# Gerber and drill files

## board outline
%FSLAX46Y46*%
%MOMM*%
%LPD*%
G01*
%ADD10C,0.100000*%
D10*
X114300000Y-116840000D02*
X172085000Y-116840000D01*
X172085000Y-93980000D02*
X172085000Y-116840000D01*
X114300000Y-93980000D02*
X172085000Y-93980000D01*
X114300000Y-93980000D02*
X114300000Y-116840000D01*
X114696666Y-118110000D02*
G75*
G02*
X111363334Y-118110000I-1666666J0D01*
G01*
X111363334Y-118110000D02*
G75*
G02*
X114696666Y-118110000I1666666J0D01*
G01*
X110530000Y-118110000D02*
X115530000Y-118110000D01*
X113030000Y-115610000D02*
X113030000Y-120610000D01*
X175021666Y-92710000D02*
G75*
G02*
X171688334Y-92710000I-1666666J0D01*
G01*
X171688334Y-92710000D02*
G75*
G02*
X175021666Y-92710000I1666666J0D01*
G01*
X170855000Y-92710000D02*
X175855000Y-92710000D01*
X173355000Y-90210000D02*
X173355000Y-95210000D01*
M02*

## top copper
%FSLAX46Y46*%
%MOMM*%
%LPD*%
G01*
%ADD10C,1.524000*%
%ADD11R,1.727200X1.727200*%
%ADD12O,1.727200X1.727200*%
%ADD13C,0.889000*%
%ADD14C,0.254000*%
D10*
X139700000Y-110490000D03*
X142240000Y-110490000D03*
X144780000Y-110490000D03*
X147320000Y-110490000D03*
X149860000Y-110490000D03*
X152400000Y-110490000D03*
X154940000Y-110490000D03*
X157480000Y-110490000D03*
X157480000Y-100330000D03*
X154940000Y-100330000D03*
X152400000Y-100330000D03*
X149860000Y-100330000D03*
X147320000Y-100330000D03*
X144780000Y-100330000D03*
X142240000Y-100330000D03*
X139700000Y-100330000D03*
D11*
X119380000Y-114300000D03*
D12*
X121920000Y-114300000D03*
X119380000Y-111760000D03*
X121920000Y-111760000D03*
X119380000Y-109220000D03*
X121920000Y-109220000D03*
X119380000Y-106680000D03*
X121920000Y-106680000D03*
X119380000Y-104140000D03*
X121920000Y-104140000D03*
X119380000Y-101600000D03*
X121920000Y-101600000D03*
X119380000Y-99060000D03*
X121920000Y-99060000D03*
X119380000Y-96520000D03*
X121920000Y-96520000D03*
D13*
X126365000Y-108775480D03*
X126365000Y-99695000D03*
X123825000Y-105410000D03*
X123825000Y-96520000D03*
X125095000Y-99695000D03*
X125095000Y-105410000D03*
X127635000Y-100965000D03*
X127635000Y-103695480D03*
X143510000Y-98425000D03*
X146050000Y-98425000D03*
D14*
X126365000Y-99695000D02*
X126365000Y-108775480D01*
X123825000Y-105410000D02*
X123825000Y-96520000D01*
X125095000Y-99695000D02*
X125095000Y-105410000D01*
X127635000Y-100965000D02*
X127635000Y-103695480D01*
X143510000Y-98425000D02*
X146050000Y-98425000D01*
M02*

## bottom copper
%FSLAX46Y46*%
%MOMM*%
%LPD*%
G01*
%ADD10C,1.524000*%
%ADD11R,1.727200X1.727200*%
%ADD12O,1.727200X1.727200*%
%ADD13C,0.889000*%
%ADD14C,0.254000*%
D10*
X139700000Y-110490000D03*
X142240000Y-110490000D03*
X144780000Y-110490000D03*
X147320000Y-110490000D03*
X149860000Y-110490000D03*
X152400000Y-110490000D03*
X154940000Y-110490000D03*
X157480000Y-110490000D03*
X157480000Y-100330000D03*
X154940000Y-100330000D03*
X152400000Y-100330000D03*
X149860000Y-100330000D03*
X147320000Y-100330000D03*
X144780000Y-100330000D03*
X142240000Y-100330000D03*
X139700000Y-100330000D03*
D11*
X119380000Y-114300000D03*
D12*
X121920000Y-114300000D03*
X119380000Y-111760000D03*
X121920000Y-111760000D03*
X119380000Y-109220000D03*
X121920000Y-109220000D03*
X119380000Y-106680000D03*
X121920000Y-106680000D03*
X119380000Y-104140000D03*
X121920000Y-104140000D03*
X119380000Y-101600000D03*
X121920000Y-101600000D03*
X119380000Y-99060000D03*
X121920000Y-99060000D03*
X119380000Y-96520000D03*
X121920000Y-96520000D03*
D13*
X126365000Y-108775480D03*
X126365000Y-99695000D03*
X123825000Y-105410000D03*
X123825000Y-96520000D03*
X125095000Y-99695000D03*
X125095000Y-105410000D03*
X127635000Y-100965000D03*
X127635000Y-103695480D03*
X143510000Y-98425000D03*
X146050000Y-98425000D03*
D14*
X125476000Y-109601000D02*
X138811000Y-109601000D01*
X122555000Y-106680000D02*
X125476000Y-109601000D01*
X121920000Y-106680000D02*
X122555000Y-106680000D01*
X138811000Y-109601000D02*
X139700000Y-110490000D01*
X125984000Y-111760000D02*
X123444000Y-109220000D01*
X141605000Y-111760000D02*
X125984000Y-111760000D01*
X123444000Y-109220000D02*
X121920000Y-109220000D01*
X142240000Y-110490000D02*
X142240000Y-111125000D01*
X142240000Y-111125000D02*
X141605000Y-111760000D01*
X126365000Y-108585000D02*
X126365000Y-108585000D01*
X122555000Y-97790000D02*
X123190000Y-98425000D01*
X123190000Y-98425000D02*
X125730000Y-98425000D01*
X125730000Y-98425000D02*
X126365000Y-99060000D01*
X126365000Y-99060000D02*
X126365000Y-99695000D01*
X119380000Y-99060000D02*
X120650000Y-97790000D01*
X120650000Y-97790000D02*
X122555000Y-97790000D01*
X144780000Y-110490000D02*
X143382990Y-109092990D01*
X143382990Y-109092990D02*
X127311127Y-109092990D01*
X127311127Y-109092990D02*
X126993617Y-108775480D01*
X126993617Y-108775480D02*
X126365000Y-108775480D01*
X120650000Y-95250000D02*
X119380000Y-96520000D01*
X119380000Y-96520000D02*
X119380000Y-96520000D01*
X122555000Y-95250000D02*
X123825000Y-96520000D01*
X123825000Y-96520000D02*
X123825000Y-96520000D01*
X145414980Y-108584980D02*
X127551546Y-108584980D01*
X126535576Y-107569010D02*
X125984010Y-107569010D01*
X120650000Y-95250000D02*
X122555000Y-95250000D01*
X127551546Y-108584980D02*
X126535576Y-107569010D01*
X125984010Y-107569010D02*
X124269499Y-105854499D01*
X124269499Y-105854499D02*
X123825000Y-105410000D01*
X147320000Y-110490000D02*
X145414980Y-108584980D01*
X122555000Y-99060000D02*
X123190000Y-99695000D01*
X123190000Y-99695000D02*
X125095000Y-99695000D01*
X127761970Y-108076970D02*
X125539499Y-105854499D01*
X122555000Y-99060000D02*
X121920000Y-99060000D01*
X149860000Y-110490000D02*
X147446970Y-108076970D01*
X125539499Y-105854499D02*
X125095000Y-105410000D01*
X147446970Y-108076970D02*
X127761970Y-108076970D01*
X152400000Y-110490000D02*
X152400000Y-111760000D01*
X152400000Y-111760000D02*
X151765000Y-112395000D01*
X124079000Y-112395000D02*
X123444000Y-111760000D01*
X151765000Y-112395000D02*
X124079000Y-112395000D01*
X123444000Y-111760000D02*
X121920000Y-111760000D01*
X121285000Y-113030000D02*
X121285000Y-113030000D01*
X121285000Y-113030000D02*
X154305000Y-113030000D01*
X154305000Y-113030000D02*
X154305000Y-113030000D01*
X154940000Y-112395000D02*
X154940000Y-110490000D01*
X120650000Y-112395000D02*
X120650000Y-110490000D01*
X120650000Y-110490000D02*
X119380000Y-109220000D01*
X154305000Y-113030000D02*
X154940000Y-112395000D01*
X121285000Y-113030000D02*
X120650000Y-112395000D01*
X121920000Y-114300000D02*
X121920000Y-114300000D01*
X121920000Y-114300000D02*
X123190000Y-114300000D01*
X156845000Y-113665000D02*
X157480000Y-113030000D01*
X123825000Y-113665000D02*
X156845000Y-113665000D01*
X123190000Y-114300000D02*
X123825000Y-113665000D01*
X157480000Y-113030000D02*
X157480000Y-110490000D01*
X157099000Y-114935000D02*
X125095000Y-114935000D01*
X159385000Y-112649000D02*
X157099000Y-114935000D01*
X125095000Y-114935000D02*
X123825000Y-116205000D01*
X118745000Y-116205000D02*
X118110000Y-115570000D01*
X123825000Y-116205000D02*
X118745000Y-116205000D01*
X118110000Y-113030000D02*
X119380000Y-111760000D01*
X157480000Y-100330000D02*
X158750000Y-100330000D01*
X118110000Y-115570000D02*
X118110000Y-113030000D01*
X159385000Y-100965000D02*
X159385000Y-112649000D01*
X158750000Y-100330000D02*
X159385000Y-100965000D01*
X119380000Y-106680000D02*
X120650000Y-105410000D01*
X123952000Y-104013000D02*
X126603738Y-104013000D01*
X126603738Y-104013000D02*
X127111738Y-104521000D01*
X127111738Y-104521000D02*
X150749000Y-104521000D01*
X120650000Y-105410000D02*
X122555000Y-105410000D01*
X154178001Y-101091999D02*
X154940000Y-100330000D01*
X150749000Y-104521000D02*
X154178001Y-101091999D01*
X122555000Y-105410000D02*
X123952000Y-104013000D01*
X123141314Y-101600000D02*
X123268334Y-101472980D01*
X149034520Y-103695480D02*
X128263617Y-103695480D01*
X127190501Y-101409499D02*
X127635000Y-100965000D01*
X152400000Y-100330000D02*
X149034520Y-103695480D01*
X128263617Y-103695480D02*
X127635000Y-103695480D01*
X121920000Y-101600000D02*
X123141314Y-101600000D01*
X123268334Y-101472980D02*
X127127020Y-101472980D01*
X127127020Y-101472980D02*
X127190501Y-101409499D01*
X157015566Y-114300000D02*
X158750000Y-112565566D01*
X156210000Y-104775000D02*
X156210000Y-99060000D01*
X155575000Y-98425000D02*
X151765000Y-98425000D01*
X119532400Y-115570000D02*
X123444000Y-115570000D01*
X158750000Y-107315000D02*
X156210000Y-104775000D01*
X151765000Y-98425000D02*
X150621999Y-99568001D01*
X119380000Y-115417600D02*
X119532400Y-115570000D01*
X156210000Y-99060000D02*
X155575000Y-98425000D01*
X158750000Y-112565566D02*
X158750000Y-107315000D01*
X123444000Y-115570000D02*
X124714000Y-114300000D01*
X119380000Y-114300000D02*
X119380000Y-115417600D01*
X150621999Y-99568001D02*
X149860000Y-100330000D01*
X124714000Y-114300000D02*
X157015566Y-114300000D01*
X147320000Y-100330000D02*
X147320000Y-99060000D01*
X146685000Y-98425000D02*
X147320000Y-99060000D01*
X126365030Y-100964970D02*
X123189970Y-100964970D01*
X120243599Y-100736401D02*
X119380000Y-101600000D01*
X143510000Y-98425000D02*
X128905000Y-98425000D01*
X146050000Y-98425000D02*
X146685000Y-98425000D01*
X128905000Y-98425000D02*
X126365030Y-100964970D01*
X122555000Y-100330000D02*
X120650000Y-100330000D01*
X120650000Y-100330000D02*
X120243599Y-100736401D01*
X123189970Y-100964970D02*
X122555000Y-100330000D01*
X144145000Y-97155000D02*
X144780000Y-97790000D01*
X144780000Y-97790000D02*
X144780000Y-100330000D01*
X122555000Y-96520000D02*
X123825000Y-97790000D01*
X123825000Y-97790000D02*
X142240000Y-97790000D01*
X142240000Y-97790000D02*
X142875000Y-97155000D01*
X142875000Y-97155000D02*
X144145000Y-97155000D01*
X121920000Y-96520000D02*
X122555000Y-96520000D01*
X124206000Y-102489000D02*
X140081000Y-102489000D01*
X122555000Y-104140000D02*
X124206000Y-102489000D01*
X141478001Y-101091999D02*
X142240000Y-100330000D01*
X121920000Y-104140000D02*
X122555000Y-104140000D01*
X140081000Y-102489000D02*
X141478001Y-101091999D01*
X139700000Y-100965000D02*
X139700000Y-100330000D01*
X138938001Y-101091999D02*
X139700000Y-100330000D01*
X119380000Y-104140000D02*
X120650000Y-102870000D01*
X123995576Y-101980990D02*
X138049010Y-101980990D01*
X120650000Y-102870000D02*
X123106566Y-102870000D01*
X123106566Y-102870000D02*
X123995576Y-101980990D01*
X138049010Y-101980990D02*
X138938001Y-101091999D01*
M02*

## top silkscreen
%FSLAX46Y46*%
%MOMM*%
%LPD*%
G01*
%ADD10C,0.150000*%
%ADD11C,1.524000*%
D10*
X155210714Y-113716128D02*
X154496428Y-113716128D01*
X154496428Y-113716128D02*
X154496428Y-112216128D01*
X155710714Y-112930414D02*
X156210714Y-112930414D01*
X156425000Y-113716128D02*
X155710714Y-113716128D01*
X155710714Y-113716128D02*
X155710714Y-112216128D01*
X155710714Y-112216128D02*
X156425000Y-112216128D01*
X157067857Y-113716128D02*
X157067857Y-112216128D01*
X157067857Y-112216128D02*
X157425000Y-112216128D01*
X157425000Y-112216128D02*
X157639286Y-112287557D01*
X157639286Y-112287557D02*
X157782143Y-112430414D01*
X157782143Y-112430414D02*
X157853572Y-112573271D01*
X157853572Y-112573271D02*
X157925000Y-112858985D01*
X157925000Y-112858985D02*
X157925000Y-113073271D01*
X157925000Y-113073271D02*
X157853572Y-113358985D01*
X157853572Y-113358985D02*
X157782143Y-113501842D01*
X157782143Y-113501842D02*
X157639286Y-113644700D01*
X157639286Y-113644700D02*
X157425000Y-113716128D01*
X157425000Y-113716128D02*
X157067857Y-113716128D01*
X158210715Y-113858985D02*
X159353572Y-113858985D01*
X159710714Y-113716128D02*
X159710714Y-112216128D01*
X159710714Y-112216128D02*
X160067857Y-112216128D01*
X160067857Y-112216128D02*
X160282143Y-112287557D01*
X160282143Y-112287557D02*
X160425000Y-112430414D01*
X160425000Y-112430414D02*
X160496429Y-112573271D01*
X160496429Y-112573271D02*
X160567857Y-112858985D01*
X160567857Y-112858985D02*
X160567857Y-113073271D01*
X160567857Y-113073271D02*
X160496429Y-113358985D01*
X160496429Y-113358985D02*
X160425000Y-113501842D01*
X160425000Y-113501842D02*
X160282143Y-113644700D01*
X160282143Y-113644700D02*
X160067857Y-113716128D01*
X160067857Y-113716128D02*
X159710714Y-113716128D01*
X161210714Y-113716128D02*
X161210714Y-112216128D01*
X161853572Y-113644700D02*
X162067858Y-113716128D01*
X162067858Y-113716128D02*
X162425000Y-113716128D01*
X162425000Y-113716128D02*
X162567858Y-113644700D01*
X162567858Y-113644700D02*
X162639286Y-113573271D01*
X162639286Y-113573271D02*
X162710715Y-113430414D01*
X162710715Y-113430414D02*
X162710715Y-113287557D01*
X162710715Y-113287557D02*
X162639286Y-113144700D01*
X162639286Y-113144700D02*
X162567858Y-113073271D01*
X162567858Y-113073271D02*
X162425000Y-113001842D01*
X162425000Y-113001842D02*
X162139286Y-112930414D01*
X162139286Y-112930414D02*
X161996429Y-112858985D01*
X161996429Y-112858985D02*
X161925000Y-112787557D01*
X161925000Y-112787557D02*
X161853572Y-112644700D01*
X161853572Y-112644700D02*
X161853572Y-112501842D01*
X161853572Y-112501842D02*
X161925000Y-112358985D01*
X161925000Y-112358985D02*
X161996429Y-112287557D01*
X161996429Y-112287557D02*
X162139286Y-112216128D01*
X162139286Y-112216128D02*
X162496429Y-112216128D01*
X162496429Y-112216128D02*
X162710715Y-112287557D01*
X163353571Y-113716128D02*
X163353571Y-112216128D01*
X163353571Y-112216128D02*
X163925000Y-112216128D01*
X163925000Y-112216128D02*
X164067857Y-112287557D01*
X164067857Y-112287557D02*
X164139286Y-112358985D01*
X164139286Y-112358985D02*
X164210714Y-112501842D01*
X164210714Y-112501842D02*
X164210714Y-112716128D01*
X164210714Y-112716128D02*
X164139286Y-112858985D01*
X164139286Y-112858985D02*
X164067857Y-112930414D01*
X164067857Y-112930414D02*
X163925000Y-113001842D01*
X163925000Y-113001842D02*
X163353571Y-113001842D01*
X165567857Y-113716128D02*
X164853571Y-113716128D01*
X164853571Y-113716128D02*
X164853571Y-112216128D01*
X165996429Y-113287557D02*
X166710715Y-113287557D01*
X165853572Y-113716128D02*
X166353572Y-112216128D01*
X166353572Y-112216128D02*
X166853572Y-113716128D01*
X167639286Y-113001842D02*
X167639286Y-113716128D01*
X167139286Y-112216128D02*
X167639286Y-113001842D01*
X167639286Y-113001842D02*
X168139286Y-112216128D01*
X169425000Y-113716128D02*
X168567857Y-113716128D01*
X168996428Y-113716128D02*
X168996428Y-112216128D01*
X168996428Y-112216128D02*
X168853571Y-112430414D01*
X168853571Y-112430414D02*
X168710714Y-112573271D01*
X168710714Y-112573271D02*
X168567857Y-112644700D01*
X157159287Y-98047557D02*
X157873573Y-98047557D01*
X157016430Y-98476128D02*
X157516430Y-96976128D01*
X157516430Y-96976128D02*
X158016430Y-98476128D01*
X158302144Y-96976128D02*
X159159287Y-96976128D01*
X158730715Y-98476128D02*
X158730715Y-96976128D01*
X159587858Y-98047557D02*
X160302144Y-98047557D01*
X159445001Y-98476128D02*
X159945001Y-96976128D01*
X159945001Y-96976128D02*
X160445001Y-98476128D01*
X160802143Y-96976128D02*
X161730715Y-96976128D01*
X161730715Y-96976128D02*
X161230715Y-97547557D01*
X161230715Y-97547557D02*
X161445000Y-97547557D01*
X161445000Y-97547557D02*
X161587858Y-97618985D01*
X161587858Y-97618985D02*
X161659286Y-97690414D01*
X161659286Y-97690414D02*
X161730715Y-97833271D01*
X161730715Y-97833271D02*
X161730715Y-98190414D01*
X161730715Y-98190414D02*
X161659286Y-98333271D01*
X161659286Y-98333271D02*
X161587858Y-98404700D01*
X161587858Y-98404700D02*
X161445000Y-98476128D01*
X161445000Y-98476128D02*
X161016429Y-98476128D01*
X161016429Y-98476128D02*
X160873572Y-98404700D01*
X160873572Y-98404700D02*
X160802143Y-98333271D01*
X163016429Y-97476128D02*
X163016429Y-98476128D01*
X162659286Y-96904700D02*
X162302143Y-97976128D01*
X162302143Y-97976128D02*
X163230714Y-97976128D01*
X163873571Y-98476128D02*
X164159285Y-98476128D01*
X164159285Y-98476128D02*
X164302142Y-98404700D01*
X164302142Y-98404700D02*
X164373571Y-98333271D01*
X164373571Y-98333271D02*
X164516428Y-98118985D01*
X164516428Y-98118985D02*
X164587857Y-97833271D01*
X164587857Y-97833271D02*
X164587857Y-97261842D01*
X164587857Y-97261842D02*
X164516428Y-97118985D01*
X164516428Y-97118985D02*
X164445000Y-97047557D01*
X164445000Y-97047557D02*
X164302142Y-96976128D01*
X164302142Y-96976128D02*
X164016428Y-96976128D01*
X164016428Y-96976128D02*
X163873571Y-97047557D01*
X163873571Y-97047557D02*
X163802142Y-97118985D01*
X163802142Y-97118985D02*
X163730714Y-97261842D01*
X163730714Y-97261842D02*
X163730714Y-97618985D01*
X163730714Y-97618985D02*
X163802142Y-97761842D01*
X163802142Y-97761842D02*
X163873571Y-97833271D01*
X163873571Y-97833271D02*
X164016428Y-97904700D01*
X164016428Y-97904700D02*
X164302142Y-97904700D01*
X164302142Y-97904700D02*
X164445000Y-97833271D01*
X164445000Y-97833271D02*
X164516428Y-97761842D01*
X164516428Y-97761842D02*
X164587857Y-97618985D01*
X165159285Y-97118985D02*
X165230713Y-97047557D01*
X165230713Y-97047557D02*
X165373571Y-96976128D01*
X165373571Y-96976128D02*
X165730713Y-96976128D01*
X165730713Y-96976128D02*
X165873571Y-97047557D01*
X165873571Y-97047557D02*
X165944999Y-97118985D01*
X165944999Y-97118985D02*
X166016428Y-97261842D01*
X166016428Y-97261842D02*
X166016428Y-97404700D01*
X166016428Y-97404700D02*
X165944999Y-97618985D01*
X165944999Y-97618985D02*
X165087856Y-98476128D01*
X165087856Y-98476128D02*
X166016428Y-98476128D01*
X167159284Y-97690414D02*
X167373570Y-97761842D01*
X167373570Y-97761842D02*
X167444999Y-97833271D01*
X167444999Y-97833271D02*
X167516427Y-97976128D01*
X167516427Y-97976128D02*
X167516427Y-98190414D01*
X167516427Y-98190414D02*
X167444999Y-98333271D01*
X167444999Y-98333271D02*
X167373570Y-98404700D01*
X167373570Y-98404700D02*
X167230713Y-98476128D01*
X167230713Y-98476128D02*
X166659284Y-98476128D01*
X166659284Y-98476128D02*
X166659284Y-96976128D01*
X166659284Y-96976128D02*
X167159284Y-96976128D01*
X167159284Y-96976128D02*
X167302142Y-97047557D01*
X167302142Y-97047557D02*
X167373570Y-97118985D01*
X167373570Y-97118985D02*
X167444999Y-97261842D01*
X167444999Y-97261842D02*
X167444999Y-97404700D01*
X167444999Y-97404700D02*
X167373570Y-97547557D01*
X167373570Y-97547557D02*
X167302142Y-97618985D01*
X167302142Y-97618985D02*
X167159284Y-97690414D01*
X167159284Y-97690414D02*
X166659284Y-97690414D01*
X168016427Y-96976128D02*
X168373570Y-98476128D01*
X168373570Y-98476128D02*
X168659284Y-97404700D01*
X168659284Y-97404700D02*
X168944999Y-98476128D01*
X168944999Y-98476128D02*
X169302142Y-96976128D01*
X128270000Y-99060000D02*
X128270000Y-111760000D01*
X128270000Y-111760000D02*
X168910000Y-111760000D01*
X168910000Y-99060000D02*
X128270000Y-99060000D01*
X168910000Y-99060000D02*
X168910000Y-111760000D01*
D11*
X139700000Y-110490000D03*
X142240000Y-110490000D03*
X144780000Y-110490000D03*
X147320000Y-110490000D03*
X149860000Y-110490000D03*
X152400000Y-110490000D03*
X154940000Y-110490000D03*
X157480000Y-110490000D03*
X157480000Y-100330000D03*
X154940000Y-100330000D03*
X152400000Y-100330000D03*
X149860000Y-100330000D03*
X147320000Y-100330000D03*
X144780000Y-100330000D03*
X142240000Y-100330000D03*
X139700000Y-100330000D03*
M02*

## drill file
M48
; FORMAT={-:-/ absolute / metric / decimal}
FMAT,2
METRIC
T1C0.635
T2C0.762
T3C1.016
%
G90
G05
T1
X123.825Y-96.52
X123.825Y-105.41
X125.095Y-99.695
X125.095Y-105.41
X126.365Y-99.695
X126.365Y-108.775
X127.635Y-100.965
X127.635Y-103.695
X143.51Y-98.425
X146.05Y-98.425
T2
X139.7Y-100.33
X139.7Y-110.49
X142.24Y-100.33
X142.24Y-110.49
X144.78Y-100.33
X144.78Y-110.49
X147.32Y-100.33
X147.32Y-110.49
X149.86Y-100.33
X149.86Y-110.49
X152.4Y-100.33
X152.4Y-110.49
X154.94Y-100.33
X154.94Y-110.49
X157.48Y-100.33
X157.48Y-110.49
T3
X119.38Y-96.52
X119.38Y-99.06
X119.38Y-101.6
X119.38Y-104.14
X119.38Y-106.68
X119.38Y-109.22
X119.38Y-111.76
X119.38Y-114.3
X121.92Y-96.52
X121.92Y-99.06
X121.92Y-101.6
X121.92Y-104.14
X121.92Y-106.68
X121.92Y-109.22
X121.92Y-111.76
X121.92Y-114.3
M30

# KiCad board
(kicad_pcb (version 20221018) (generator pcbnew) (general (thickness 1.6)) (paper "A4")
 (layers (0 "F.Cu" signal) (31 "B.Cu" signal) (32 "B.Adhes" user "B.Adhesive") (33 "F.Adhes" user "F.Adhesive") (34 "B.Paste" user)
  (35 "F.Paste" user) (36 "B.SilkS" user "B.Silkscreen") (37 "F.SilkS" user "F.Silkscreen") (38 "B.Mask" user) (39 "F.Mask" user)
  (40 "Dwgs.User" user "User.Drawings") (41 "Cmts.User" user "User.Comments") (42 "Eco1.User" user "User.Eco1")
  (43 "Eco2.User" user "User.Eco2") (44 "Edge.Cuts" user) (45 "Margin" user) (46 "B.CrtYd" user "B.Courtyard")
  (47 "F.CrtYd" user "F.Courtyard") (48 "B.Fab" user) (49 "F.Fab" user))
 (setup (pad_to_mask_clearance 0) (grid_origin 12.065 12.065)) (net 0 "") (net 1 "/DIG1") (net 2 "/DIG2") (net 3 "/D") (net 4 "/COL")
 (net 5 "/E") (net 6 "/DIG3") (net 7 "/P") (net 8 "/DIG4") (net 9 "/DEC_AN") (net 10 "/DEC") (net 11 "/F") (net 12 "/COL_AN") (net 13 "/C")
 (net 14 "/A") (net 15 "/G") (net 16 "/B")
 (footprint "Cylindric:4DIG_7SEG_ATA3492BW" (layer "F.Cu") (at 148.59 105.41)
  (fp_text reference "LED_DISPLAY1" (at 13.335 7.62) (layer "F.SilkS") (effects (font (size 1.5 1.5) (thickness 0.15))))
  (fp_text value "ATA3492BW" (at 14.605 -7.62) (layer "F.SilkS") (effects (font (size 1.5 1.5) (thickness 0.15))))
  (fp_line (start -20.32 -6.35) (end -20.32 6.35) (stroke (width 0.15) (type solid)) (layer "F.SilkS"))
  (fp_line (start -20.32 6.35) (end 20.32 6.35) (stroke (width 0.15) (type solid)) (layer "F.SilkS"))
  (fp_line (start 20.32 -6.35) (end -20.32 -6.35) (stroke (width 0.15) (type solid)) (layer "F.SilkS"))
  (fp_line (start 20.32 -6.35) (end 20.32 6.35) (stroke (width 0.15) (type solid)) (layer "F.SilkS"))
  (pad "1" thru_hole circle (at -8.89 5.08) (size 1.524 1.524) (drill 0.762) (layers "*.Cu" "*.Mask" "F.SilkS") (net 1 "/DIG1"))
  (pad "2" thru_hole circle (at -6.35 5.08) (size 1.524 1.524) (drill 0.762) (layers "*.Cu" "*.Mask" "F.SilkS") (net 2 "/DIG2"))
  (pad "3" thru_hole circle (at -3.81 5.08) (size 1.524 1.524) (drill 0.762) (layers "*.Cu" "*.Mask" "F.SilkS") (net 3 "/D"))
  (pad "4" thru_hole circle (at -1.27 5.08) (size 1.524 1.524) (drill 0.762) (layers "*.Cu" "*.Mask" "F.SilkS") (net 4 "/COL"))
  (pad "5" thru_hole circle (at 1.27 5.08) (size 1.524 1.524) (drill 0.762) (layers "*.Cu" "*.Mask" "F.SilkS") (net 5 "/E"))
  (pad "6" thru_hole circle (at 3.81 5.08) (size 1.524 1.524) (drill 0.762) (layers "*.Cu" "*.Mask" "F.SilkS") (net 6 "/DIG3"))
  (pad "7" thru_hole circle (at 6.35 5.08) (size 1.524 1.524) (drill 0.762) (layers "*.Cu" "*.Mask" "F.SilkS") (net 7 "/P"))
  (pad "8" thru_hole circle (at 8.89 5.08) (size 1.524 1.524) (drill 0.762) (layers "*.Cu" "*.Mask" "F.SilkS") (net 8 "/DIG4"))
  (pad "9" thru_hole circle (at 8.89 -5.08) (size 1.524 1.524) (drill 0.762) (layers "*.Cu" "*.Mask" "F.SilkS") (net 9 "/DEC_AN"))
  (pad "10" thru_hole circle (at 6.35 -5.08) (size 1.524 1.524) (drill 0.762) (layers "*.Cu" "*.Mask" "F.SilkS") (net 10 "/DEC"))
  (pad "11" thru_hole circle (at 3.81 -5.08) (size 1.524 1.524) (drill 0.762) (layers "*.Cu" "*.Mask" "F.SilkS") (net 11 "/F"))
  (pad "12" thru_hole circle (at 1.27 -5.08) (size 1.524 1.524) (drill 0.762) (layers "*.Cu" "*.Mask" "F.SilkS") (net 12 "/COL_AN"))
  (pad "13" thru_hole circle (at -1.27 -5.08) (size 1.524 1.524) (drill 0.762) (layers "*.Cu" "*.Mask" "F.SilkS") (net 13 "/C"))
  (pad "14" thru_hole circle (at -3.81 -5.08) (size 1.524 1.524) (drill 0.762) (layers "*.Cu" "*.Mask" "F.SilkS") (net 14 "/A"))
  (pad "15" thru_hole circle (at -6.35 -5.08) (size 1.524 1.524) (drill 0.762) (layers "*.Cu" "*.Mask" "F.SilkS") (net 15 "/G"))
  (pad "16" thru_hole circle (at -8.89 -5.08) (size 1.524 1.524) (drill 0.762) (layers "*.Cu" "*.Mask" "F.SilkS") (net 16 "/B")))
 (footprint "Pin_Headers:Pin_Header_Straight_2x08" (layer "B.Cu") (at 120.65 105.41 90)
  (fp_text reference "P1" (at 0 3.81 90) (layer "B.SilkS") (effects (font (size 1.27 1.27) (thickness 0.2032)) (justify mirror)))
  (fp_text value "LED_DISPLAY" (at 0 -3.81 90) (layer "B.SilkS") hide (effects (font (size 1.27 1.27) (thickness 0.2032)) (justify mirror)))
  (pad "1" thru_hole rect (at -8.89 -1.27 90) (size 1.7272 1.7272) (drill 1.016) (layers "*.Cu" "*.Mask" "B.SilkS") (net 12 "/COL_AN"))
  (pad "2" thru_hole oval (at -8.89 1.27 90) (size 1.7272 1.7272) (drill 1.016) (layers "*.Cu" "*.Mask" "B.SilkS") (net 8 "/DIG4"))
  (pad "3" thru_hole oval (at -6.35 -1.27 90) (size 1.7272 1.7272) (drill 1.016) (layers "*.Cu" "*.Mask" "B.SilkS") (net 9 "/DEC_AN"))
  (pad "4" thru_hole oval (at -6.35 1.27 90) (size 1.7272 1.7272) (drill 1.016) (layers "*.Cu" "*.Mask" "B.SilkS") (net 6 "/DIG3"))
  (pad "5" thru_hole oval (at -3.81 -1.27 90) (size 1.7272 1.7272) (drill 1.016) (layers "*.Cu" "*.Mask" "B.SilkS") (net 7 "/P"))
  (pad "6" thru_hole oval (at -3.81 1.27 90) (size 1.7272 1.7272) (drill 1.016) (layers "*.Cu" "*.Mask" "B.SilkS") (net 2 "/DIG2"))
  (pad "7" thru_hole oval (at -1.27 -1.27 90) (size 1.7272 1.7272) (drill 1.016) (layers "*.Cu" "*.Mask" "B.SilkS") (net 10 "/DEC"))
  (pad "8" thru_hole oval (at -1.27 1.27 90) (size 1.7272 1.7272) (drill 1.016) (layers "*.Cu" "*.Mask" "B.SilkS") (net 1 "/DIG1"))
  (pad "9" thru_hole oval (at 1.27 -1.27 90) (size 1.7272 1.7272) (drill 1.016) (layers "*.Cu" "*.Mask" "B.SilkS") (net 16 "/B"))
  (pad "10" thru_hole oval (at 1.27 1.27 90) (size 1.7272 1.7272) (drill 1.016) (layers "*.Cu" "*.Mask" "B.SilkS") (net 15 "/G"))
  (pad "11" thru_hole oval (at 3.81 -1.27 90) (size 1.7272 1.7272) (drill 1.016) (layers "*.Cu" "*.Mask" "B.SilkS") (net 13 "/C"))
  (pad "12" thru_hole oval (at 3.81 1.27 90) (size 1.7272 1.7272) (drill 1.016) (layers "*.Cu" "*.Mask" "B.SilkS") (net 11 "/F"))
  (pad "13" thru_hole oval (at 6.35 -1.27 90) (size 1.7272 1.7272) (drill 1.016) (layers "*.Cu" "*.Mask" "B.SilkS") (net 3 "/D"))
  (pad "14" thru_hole oval (at 6.35 1.27 90) (size 1.7272 1.7272) (drill 1.016) (layers "*.Cu" "*.Mask" "B.SilkS") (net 5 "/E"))
  (pad "15" thru_hole oval (at 8.89 -1.27 90) (size 1.7272 1.7272) (drill 1.016) (layers "*.Cu" "*.Mask" "B.SilkS") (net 4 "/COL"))
  (pad "16" thru_hole oval (at 8.89 1.27 90) (size 1.7272 1.7272) (drill 1.016) (layers "*.Cu" "*.Mask" "B.SilkS") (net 14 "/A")))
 (gr_line (start 114.3 116.84) (end 172.085 116.84) (stroke (width 0.1) (type solid)) (layer "Edge.Cuts"))
 (gr_line (start 172.085 93.98) (end 172.085 116.84) (stroke (width 0.1) (type solid)) (layer "Edge.Cuts"))
 (gr_line (start 114.3 93.98) (end 172.085 93.98) (stroke (width 0.1) (type solid)) (layer "Edge.Cuts"))
 (gr_line (start 114.3 93.98) (end 114.3 116.84) (stroke (width 0.1) (type solid)) (layer "Edge.Cuts"))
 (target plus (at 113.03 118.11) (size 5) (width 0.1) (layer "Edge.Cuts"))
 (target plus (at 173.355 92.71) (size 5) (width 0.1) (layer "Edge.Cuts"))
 (segment (start 125.476 109.601) (end 138.811 109.601) (width 0.254) (layer "B.Cu") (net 1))
 (segment (start 122.555 106.68) (end 125.476 109.601) (width 0.254) (layer "B.Cu") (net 1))
 (segment (start 121.92 106.68) (end 122.555 106.68) (width 0.254) (layer "B.Cu") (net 1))
 (segment (start 138.811 109.601) (end 139.7 110.49) (width 0.254) (layer "B.Cu") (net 1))
 (segment (start 125.984 111.76) (end 123.444 109.22) (width 0.254) (layer "B.Cu") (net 2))
 (segment (start 141.605 111.76) (end 125.984 111.76) (width 0.254) (layer "B.Cu") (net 2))
 (segment (start 123.444 109.22) (end 121.92 109.22) (width 0.254) (layer "B.Cu") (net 2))
 (segment (start 142.24 110.49) (end 142.24 111.125) (width 0.254) (layer "B.Cu") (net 2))
 (segment (start 142.24 111.125) (end 141.605 111.76) (width 0.254) (layer "B.Cu") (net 2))
 (segment (start 126.365 99.695) (end 126.365 108.77548) (width 0.254) (layer "F.Cu") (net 3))
 (via (at 126.365 108.77548) (size 0.889) (drill 0.635) (layers "F.Cu" "B.Cu") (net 3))
 (via (at 126.365 99.695) (size 0.889) (drill 0.635) (layers "F.Cu" "B.Cu") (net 3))
 (segment (start 126.365 108.585) (end 126.365 108.585) (width 0.254) (layer "B.Cu") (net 3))
 (segment (start 122.555 97.79) (end 123.19 98.425) (width 0.254) (layer "B.Cu") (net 3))
 (segment (start 123.19 98.425) (end 125.73 98.425) (width 0.254) (layer "B.Cu") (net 3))
 (segment (start 125.73 98.425) (end 126.365 99.06) (width 0.254) (layer "B.Cu") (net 3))
 (segment (start 126.365 99.06) (end 126.365 99.695) (width 0.254) (layer "B.Cu") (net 3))
 (segment (start 119.38 99.06) (end 120.65 97.79) (width 0.254) (layer "B.Cu") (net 3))
 (segment (start 120.65 97.79) (end 122.555 97.79) (width 0.254) (layer "B.Cu") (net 3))
 (segment (start 144.78 110.49) (end 143.38299 109.09299) (width 0.254) (layer "B.Cu") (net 3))
 (segment (start 143.38299 109.09299) (end 127.311127 109.09299) (width 0.254) (layer "B.Cu") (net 3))
 (segment (start 127.311127 109.09299) (end 126.993617 108.77548) (width 0.254) (layer "B.Cu") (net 3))
 (segment (start 126.993617 108.77548) (end 126.365 108.77548) (width 0.254) (layer "B.Cu") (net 3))
 (segment (start 123.825 105.41) (end 123.825 96.52) (width 0.254) (layer "F.Cu") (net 4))
 (via (at 123.825 105.41) (size 0.889) (drill 0.635) (layers "F.Cu" "B.Cu") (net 4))
 (via (at 123.825 96.52) (size 0.889) (drill 0.635) (layers "F.Cu" "B.Cu") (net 4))
 (segment (start 120.65 95.25) (end 119.38 96.52) (width 0.254) (layer "B.Cu") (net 4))
 (segment (start 119.38 96.52) (end 119.38 96.52) (width 0.254) (layer "B.Cu") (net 4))
 (segment (start 122.555 95.25) (end 123.825 96.52) (width 0.254) (layer "B.Cu") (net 4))
 (segment (start 123.825 96.52) (end 123.825 96.52) (width 0.254) (layer "B.Cu") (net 4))
 (segment (start 145.41498 108.58498) (end 127.551546 108.58498) (width 0.254) (layer "B.Cu") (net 4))
 (segment (start 126.535576 107.56901) (end 125.98401 107.56901) (width 0.254) (layer "B.Cu") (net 4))
 (segment (start 120.65 95.25) (end 122.555 95.25) (width 0.254) (layer "B.Cu") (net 4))
 (segment (start 127.551546 108.58498) (end 126.535576 107.56901) (width 0.254) (layer "B.Cu") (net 4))
 (segment (start 125.98401 107.56901) (end 124.269499 105.854499) (width 0.254) (layer "B.Cu") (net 4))
 (segment (start 124.269499 105.854499) (end 123.825 105.41) (width 0.254) (layer "B.Cu") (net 4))
 (segment (start 147.32 110.49) (end 145.41498 108.58498) (width 0.254) (layer "B.Cu") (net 4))
 (segment (start 125.095 99.695) (end 125.095 105.41) (width 0.254) (layer "F.Cu") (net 5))
 (via (at 125.095 99.695) (size 0.889) (drill 0.635) (layers "F.Cu" "B.Cu") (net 5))
 (via (at 125.095 105.41) (size 0.889) (drill 0.635) (layers "F.Cu" "B.Cu") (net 5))
 (segment (start 122.555 99.06) (end 123.19 99.695) (width 0.254) (layer "B.Cu") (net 5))
 (segment (start 123.19 99.695) (end 125.095 99.695) (width 0.254) (layer "B.Cu") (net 5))
 (segment (start 127.76197 108.07697) (end 125.539499 105.854499) (width 0.254) (layer "B.Cu") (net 5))
 (segment (start 122.555 99.06) (end 121.92 99.06) (width 0.254) (layer "B.Cu") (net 5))
 (segment (start 149.86 110.49) (end 147.44697 108.07697) (width 0.254) (layer "B.Cu") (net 5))
 (segment (start 125.539499 105.854499) (end 125.095 105.41) (width 0.254) (layer "B.Cu") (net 5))
 (segment (start 147.44697 108.07697) (end 127.76197 108.07697) (width 0.254) (layer "B.Cu") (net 5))
 (segment (start 152.4 110.49) (end 152.4 111.76) (width 0.254) (layer "B.Cu") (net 6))
 (segment (start 152.4 111.76) (end 151.765 112.395) (width 0.254) (layer "B.Cu") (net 6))
 (segment (start 124.079 112.395) (end 123.444 111.76) (width 0.254) (layer "B.Cu") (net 6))
 (segment (start 151.765 112.395) (end 124.079 112.395) (width 0.254) (layer "B.Cu") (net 6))
 (segment (start 123.444 111.76) (end 121.92 111.76) (width 0.254) (layer "B.Cu") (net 6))
 (segment (start 121.285 113.03) (end 121.285 113.03) (width 0.254) (layer "B.Cu") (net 7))
 (segment (start 121.285 113.03) (end 154.305 113.03) (width 0.254) (layer "B.Cu") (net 7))
 (segment (start 154.305 113.03) (end 154.305 113.03) (width 0.254) (layer "B.Cu") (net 7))
 (segment (start 154.94 112.395) (end 154.94 110.49) (width 0.254) (layer "B.Cu") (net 7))
 (segment (start 120.65 112.395) (end 120.65 110.49) (width 0.254) (layer "B.Cu") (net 7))
 (segment (start 120.65 110.49) (end 119.38 109.22) (width 0.254) (layer "B.Cu") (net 7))
 (segment (start 154.305 113.03) (end 154.94 112.395) (width 0.254) (layer "B.Cu") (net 7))
 (segment (start 121.285 113.03) (end 120.65 112.395) (width 0.254) (layer "B.Cu") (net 7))
 (segment (start 121.92 114.3) (end 121.92 114.3) (width 0.254) (layer "B.Cu") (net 8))
 (segment (start 121.92 114.3) (end 123.19 114.3) (width 0.254) (layer "B.Cu") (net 8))
 (segment (start 156.845 113.665) (end 157.48 113.03) (width 0.254) (layer "B.Cu") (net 8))
 (segment (start 123.825 113.665) (end 156.845 113.665) (width 0.254) (layer "B.Cu") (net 8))
 (segment (start 123.19 114.3) (end 123.825 113.665) (width 0.254) (layer "B.Cu") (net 8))
 (segment (start 157.48 113.03) (end 157.48 110.49) (width 0.254) (layer "B.Cu") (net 8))
 (segment (start 157.099 114.935) (end 125.095 114.935) (width 0.254) (layer "B.Cu") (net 9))
 (segment (start 159.385 112.649) (end 157.099 114.935) (width 0.254) (layer "B.Cu") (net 9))
 (segment (start 125.095 114.935) (end 123.825 116.205) (width 0.254) (layer "B.Cu") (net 9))
 (segment (start 118.745 116.205) (end 118.11 115.57) (width 0.254) (layer "B.Cu") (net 9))
 (segment (start 123.825 116.205) (end 118.745 116.205) (width 0.254) (layer "B.Cu") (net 9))
 (segment (start 118.11 113.03) (end 119.38 111.76) (width 0.254) (layer "B.Cu") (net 9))
 (segment (start 157.48 100.33) (end 158.75 100.33) (width 0.254) (layer "B.Cu") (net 9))
 (segment (start 118.11 115.57) (end 118.11 113.03) (width 0.254) (layer "B.Cu") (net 9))
 (segment (start 159.385 100.965) (end 159.385 112.649) (width 0.254) (layer "B.Cu") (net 9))
 (segment (start 158.75 100.33) (end 159.385 100.965) (width 0.254) (layer "B.Cu") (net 9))
 (segment (start 119.38 106.68) (end 120.65 105.41) (width 0.254) (layer "B.Cu") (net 10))
 (segment (start 123.952 104.013) (end 126.603738 104.013) (width 0.254) (layer "B.Cu") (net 10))
 (segment (start 126.603738 104.013) (end 127.111738 104.521) (width 0.254) (layer "B.Cu") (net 10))
 (segment (start 127.111738 104.521) (end 150.749 104.521) (width 0.254) (layer "B.Cu") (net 10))
 (segment (start 120.65 105.41) (end 122.555 105.41) (width 0.254) (layer "B.Cu") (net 10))
 (segment (start 154.178001 101.091999) (end 154.94 100.33) (width 0.254) (layer "B.Cu") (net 10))
 (segment (start 150.749 104.521) (end 154.178001 101.091999) (width 0.254) (layer "B.Cu") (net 10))
 (segment (start 122.555 105.41) (end 123.952 104.013) (width 0.254) (layer "B.Cu") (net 10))
 (segment (start 127.635 100.965) (end 127.635 103.69548) (width 0.254) (layer "F.Cu") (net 11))
 (via (at 127.635 100.965) (size 0.889) (drill 0.635) (layers "F.Cu" "B.Cu") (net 11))
 (via (at 127.635 103.69548) (size 0.889) (drill 0.635) (layers "F.Cu" "B.Cu") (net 11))
 (segment (start 123.141314 101.6) (end 123.268334 101.47298) (width 0.254) (layer "B.Cu") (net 11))
 (segment (start 149.03452 103.69548) (end 128.263617 103.69548) (width 0.254) (layer "B.Cu") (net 11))
 (segment (start 127.190501 101.409499) (end 127.635 100.965) (width 0.254) (layer "B.Cu") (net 11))
 (segment (start 152.4 100.33) (end 149.03452 103.69548) (width 0.254) (layer "B.Cu") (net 11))
 (segment (start 128.263617 103.69548) (end 127.635 103.69548) (width 0.254) (layer "B.Cu") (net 11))
 (segment (start 121.92 101.6) (end 123.141314 101.6) (width 0.254) (layer "B.Cu") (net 11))
 (segment (start 123.268334 101.47298) (end 127.12702 101.47298) (width 0.254) (layer "B.Cu") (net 11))
 (segment (start 127.12702 101.47298) (end 127.190501 101.409499) (width 0.254) (layer "B.Cu") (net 11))
 (segment (start 157.015566 114.3) (end 158.75 112.565566) (width 0.254) (layer "B.Cu") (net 12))
 (segment (start 156.21 104.775) (end 156.21 99.06) (width 0.254) (layer "B.Cu") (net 12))
 (segment (start 155.575 98.425) (end 151.765 98.425) (width 0.254) (layer "B.Cu") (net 12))
 (segment (start 119.5324 115.57) (end 123.444 115.57) (width 0.254) (layer "B.Cu") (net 12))
 (segment (start 158.75 107.315) (end 156.21 104.775) (width 0.254) (layer "B.Cu") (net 12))
 (segment (start 151.765 98.425) (end 150.621999 99.568001) (width 0.254) (layer "B.Cu") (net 12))
 (segment (start 119.38 115.4176) (end 119.5324 115.57) (width 0.254) (layer "B.Cu") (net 12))
 (segment (start 156.21 99.06) (end 155.575 98.425) (width 0.254) (layer "B.Cu") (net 12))
 (segment (start 158.75 112.565566) (end 158.75 107.315) (width 0.254) (layer "B.Cu") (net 12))
 (segment (start 123.444 115.57) (end 124.714 114.3) (width 0.254) (layer "B.Cu") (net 12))
 (segment (start 119.38 114.3) (end 119.38 115.4176) (width 0.254) (layer "B.Cu") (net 12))
 (segment (start 150.621999 99.568001) (end 149.86 100.33) (width 0.254) (layer "B.Cu") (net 12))
 (segment (start 124.714 114.3) (end 157.015566 114.3) (width 0.254) (layer "B.Cu") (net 12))
 (segment (start 143.51 98.425) (end 146.05 98.425) (width 0.254) (layer "F.Cu") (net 13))
 (via (at 143.51 98.425) (size 0.889) (drill 0.635) (layers "F.Cu" "B.Cu") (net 13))
 (via (at 146.05 98.425) (size 0.889) (drill 0.635) (layers "F.Cu" "B.Cu") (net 13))
 (segment (start 147.32 100.33) (end 147.32 99.06) (width 0.254) (layer "B.Cu") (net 13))
 (segment (start 146.685 98.425) (end 147.32 99.06) (width 0.254) (layer "B.Cu") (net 13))
 (segment (start 126.36503 100.96497) (end 123.18997 100.96497) (width 0.254) (layer "B.Cu") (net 13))
 (segment (start 120.243599 100.736401) (end 119.38 101.6) (width 0.254) (layer "B.Cu") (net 13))
 (segment (start 143.51 98.425) (end 128.905 98.425) (width 0.254) (layer "B.Cu") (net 13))
 (segment (start 146.05 98.425) (end 146.685 98.425) (width 0.254) (layer "B.Cu") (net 13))
 (segment (start 128.905 98.425) (end 126.36503 100.96497) (width 0.254) (layer "B.Cu") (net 13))
 (segment (start 122.555 100.33) (end 120.65 100.33) (width 0.254) (layer "B.Cu") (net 13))
 (segment (start 120.65 100.33) (end 120.243599 100.736401) (width 0.254) (layer "B.Cu") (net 13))
 (segment (start 123.18997 100.96497) (end 122.555 100.33) (width 0.254) (layer "B.Cu") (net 13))
 (segment (start 144.145 97.155) (end 144.78 97.79) (width 0.254) (layer "B.Cu") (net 14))
 (segment (start 144.78 97.79) (end 144.78 100.33) (width 0.254) (layer "B.Cu") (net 14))
 (segment (start 122.555 96.52) (end 123.825 97.79) (width 0.254) (layer "B.Cu") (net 14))
 (segment (start 123.825 97.79) (end 142.24 97.79) (width 0.254) (layer "B.Cu") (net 14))
 (segment (start 142.24 97.79) (end 142.875 97.155) (width 0.254) (layer "B.Cu") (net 14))
 (segment (start 142.875 97.155) (end 144.145 97.155) (width 0.254) (layer "B.Cu") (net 14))
 (segment (start 121.92 96.52) (end 122.555 96.52) (width 0.254) (layer "B.Cu") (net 14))
 (segment (start 124.206 102.489) (end 140.081 102.489) (width 0.254) (layer "B.Cu") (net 15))
 (segment (start 122.555 104.14) (end 124.206 102.489) (width 0.254) (layer "B.Cu") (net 15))
 (segment (start 141.478001 101.091999) (end 142.24 100.33) (width 0.254) (layer "B.Cu") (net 15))
 (segment (start 121.92 104.14) (end 122.555 104.14) (width 0.254) (layer "B.Cu") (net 15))
 (segment (start 140.081 102.489) (end 141.478001 101.091999) (width 0.254) (layer "B.Cu") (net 15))
 (segment (start 139.7 100.965) (end 139.7 100.33) (width 0.254) (layer "B.Cu") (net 16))
 (segment (start 138.938001 101.091999) (end 139.7 100.33) (width 0.254) (layer "B.Cu") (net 16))
 (segment (start 119.38 104.14) (end 120.65 102.87) (width 0.254) (layer "B.Cu") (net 16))
 (segment (start 123.995576 101.98099) (end 138.04901 101.98099) (width 0.254) (layer "B.Cu") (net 16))
 (segment (start 120.65 102.87) (end 123.106566 102.87) (width 0.254) (layer "B.Cu") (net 16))
 (segment (start 123.106566 102.87) (end 123.995576 101.98099) (width 0.254) (layer "B.Cu") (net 16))
 (segment (start 138.04901 101.98099) (end 138.938001 101.091999) (width 0.254) (layer "B.Cu") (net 16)))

